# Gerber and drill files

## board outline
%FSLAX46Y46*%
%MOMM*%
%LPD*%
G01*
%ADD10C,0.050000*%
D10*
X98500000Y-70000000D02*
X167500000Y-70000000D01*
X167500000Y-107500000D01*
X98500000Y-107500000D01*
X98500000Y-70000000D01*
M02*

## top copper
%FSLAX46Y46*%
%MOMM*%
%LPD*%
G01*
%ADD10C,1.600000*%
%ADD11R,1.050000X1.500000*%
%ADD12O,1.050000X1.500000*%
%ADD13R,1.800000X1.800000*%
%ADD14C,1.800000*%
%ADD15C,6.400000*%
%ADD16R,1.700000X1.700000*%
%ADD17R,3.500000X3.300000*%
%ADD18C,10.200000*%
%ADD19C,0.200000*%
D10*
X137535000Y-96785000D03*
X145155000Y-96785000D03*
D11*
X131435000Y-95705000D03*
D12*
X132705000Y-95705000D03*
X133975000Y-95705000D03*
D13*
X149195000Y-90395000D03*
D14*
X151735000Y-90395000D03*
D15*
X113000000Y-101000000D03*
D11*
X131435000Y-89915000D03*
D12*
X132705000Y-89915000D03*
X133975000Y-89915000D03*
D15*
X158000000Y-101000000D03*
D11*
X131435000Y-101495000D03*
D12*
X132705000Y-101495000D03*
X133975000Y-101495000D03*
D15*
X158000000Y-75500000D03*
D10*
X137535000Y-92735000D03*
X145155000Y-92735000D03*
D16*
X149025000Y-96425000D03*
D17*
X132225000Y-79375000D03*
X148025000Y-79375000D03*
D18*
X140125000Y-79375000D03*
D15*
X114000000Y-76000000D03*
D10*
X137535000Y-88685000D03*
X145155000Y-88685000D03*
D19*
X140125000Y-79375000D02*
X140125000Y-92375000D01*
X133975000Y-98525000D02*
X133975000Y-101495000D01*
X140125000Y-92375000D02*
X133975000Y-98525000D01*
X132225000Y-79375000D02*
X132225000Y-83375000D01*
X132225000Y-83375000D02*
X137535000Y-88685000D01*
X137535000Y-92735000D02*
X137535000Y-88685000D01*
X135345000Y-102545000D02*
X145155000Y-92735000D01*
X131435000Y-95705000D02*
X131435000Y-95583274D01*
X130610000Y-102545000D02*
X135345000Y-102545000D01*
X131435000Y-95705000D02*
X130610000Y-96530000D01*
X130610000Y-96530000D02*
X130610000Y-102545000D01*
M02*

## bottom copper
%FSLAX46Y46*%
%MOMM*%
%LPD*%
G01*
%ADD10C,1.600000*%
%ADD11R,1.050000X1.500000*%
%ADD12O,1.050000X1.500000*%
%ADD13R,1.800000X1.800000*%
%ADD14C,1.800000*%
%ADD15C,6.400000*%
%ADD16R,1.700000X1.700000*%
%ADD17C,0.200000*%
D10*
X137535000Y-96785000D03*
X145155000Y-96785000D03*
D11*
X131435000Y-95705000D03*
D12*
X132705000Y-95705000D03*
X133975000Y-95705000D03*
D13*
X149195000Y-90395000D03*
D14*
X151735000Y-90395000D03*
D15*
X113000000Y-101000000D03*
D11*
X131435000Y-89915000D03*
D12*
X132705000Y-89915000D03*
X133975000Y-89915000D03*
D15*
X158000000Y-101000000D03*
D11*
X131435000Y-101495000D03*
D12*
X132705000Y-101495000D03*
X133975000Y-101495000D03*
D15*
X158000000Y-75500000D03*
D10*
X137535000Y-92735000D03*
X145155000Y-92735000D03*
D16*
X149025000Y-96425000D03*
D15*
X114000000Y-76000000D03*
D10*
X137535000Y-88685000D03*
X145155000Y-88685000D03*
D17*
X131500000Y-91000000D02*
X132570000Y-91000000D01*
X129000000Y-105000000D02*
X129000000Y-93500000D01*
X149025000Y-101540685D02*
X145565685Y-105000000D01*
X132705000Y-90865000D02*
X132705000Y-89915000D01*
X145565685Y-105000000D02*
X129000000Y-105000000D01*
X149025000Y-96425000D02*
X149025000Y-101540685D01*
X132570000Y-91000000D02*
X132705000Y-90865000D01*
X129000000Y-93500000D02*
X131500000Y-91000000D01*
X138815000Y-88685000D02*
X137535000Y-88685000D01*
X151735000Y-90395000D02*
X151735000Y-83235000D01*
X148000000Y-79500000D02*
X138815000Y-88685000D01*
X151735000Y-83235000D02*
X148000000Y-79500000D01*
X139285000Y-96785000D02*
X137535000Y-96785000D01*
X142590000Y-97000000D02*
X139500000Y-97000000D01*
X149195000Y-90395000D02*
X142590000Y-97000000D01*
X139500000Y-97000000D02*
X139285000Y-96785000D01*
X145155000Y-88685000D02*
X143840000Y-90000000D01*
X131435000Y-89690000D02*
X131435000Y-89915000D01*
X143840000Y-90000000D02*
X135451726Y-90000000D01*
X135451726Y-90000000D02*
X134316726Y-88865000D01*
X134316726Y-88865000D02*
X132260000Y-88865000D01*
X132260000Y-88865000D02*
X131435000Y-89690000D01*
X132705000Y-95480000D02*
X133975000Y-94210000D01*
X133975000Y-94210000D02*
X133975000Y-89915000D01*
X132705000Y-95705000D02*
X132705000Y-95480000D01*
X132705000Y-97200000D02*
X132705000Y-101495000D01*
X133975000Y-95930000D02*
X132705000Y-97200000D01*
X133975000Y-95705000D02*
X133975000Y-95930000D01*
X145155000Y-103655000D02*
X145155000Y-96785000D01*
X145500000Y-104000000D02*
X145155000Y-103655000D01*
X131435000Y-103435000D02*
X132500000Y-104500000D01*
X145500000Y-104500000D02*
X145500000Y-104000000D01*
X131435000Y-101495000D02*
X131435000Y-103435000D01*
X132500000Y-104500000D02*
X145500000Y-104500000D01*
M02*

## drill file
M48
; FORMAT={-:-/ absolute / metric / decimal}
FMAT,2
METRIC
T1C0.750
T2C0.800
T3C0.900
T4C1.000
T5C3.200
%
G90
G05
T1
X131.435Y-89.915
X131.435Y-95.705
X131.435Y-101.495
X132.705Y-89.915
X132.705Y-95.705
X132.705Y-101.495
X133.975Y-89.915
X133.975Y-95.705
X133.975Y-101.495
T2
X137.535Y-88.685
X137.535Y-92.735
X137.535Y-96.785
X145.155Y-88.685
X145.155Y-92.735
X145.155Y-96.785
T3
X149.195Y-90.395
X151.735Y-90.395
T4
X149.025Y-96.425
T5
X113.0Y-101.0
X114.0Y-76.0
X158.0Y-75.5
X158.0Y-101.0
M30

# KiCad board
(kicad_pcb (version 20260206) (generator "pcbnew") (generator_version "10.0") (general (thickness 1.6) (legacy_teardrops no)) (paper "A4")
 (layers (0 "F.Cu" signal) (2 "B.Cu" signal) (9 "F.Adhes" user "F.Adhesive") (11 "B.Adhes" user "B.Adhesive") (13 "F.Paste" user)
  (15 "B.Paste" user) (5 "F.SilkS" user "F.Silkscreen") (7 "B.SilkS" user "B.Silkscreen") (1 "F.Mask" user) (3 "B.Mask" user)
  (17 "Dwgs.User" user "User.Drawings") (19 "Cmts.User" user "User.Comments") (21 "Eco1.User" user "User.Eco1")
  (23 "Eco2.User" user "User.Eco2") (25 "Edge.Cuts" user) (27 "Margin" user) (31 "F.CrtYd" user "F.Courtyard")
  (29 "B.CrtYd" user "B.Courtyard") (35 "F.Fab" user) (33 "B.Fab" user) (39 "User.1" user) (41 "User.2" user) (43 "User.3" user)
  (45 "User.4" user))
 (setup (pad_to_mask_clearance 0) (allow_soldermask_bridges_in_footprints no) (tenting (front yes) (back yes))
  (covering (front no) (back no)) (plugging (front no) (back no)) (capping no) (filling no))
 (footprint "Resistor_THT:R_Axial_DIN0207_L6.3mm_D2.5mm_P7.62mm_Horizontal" (layer "F.Cu") (at 137.535 96.785)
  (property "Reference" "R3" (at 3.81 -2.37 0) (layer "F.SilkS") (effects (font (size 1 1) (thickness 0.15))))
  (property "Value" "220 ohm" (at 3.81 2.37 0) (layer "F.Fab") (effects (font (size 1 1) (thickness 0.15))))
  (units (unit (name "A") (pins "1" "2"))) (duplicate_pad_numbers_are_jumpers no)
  (pad "1" thru_hole circle (at 0 0) (size 1.6 1.6) (drill 0.8) (layers "*.Cu" "*.Mask") (remove_unused_layers no) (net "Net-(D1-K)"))
  (pad "2" thru_hole circle (at 7.62 0) (size 1.6 1.6) (drill 0.8) (layers "*.Cu" "*.Mask") (remove_unused_layers no) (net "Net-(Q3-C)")))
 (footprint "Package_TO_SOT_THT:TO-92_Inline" (layer "F.Cu") (at 131.435 95.705)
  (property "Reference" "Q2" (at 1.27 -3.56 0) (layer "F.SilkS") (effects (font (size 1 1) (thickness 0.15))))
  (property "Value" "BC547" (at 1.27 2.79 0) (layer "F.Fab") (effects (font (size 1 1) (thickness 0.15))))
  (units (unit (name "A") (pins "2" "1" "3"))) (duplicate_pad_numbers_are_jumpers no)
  (pad "1" thru_hole rect (at 0 0) (size 1.05 1.5) (drill 0.75) (layers "*.Cu" "*.Mask") (remove_unused_layers no) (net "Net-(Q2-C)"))
  (pad "2" thru_hole oval (at 1.27 0) (size 1.05 1.5) (drill 0.75) (layers "*.Cu" "*.Mask") (remove_unused_layers no) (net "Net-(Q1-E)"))
  (pad "3" thru_hole oval (at 2.54 0) (size 1.05 1.5) (drill 0.75) (layers "*.Cu" "*.Mask") (remove_unused_layers no) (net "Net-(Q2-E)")))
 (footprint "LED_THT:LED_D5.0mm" (layer "F.Cu") (at 149.195 90.395)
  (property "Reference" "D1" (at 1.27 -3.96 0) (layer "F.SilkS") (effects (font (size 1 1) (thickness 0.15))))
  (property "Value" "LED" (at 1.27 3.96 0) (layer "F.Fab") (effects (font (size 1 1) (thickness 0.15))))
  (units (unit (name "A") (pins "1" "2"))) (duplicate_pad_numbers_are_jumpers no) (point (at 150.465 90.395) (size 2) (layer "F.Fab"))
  (pad "1" thru_hole rect (at 0 0) (size 1.8 1.8) (drill 0.9) (layers "*.Cu" "*.Mask") (remove_unused_layers no) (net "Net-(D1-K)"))
  (pad "2" thru_hole circle (at 2.54 0) (size 1.8 1.8) (drill 0.9) (layers "*.Cu" "*.Mask") (remove_unused_layers no) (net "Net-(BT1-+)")))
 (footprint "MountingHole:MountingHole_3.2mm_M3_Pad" (layer "F.Cu") (at 113 101)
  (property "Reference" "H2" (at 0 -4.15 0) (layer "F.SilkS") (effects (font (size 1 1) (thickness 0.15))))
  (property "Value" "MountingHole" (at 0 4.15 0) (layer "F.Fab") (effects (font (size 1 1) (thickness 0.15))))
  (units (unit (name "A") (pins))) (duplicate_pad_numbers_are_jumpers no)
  (pad "1" thru_hole circle (at 0 0) (size 6.4 6.4) (drill 3.2) (layers "*.Cu" "*.Mask") (remove_unused_layers no) (zone_connect 2)))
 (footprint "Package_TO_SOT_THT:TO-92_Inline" (layer "F.Cu") (at 131.435 89.915)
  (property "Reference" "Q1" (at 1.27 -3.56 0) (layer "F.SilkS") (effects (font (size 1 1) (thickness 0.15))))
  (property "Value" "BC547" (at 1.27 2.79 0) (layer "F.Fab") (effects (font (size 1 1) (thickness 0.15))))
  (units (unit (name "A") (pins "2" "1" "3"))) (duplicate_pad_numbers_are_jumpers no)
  (pad "1" thru_hole rect (at 0 0) (size 1.05 1.5) (drill 0.75) (layers "*.Cu" "*.Mask") (remove_unused_layers no) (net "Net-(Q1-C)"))
  (pad "2" thru_hole oval (at 1.27 0) (size 1.05 1.5) (drill 0.75) (layers "*.Cu" "*.Mask") (remove_unused_layers no) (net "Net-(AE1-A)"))
  (pad "3" thru_hole oval (at 2.54 0) (size 1.05 1.5) (drill 0.75) (layers "*.Cu" "*.Mask") (remove_unused_layers no) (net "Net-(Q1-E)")))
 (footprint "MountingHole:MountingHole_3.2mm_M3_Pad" (layer "F.Cu") (at 158 101)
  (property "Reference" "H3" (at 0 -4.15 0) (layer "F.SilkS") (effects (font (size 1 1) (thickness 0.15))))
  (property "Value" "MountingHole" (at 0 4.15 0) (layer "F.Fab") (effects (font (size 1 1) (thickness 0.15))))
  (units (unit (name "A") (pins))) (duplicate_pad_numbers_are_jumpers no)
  (pad "1" thru_hole circle (at 0 0) (size 6.4 6.4) (drill 3.2) (layers "*.Cu" "*.Mask") (remove_unused_layers no) (zone_connect 2)))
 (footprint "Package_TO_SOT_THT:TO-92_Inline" (layer "F.Cu") (at 131.435 101.495)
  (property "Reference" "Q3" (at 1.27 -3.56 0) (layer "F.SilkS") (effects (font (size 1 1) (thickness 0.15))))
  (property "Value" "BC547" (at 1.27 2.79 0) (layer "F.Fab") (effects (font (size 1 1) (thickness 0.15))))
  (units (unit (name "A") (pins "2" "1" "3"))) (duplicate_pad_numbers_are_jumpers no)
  (pad "1" thru_hole rect (at 0 0) (size 1.05 1.5) (drill 0.75) (layers "*.Cu" "*.Mask") (remove_unused_layers no) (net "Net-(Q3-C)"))
  (pad "2" thru_hole oval (at 1.27 0) (size 1.05 1.5) (drill 0.75) (layers "*.Cu" "*.Mask") (remove_unused_layers no) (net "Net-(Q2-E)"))
  (pad "3" thru_hole oval (at 2.54 0) (size 1.05 1.5) (drill 0.75) (layers "*.Cu" "*.Mask") (remove_unused_layers no) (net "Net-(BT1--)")))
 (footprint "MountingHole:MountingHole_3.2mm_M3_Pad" (layer "F.Cu") (at 158 75.5)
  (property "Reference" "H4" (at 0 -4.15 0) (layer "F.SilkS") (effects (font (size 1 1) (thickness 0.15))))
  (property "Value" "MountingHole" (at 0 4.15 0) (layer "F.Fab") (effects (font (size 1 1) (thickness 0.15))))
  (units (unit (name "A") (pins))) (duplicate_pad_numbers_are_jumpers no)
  (pad "1" thru_hole circle (at 0 0) (size 6.4 6.4) (drill 3.2) (layers "*.Cu" "*.Mask") (remove_unused_layers no) (zone_connect 2)))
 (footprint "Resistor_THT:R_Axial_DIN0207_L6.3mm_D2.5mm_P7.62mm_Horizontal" (layer "F.Cu") (at 137.535 92.735)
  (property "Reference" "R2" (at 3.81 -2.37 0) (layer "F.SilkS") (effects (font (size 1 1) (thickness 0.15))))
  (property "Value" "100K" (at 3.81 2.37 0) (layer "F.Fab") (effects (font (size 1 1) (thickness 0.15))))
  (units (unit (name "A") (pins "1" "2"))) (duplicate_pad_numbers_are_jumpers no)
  (pad "1" thru_hole circle (at 0 0) (size 1.6 1.6) (drill 0.8) (layers "*.Cu" "*.Mask") (remove_unused_layers no) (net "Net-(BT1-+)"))
  (pad "2" thru_hole circle (at 7.62 0) (size 1.6 1.6) (drill 0.8) (layers "*.Cu" "*.Mask") (remove_unused_layers no) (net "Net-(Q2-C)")))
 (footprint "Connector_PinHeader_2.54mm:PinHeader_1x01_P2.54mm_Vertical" (layer "F.Cu") (at 149.025 96.425)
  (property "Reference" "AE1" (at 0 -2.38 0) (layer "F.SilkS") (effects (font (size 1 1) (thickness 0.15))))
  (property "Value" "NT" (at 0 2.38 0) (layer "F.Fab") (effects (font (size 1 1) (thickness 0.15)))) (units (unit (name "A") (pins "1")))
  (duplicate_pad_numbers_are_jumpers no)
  (pad "1" thru_hole rect (at 0 0) (size 1.7 1.7) (drill 1) (layers "*.Cu" "*.Mask") (remove_unused_layers no) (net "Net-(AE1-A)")))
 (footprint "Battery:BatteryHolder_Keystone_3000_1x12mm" (layer "F.Cu") (at 140.125 79.375)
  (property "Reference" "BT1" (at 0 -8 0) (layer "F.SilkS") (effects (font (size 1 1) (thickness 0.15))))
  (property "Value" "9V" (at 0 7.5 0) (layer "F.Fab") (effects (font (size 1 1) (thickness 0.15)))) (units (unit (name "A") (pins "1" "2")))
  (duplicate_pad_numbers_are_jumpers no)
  (pad "1" smd rect (at -7.9 0) (size 3.5 3.3) (layers "F.Cu" "F.Mask" "F.Paste") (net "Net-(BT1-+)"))
  (pad "1" smd rect (at 7.9 0) (size 3.5 3.3) (layers "F.Cu" "F.Mask" "F.Paste") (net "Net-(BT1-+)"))
  (pad "2" smd circle (at 0 0) (size 10.2 10.2) (layers "F.Cu" "F.Mask") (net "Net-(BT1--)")))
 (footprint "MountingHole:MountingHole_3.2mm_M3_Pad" (layer "F.Cu") (at 114 76)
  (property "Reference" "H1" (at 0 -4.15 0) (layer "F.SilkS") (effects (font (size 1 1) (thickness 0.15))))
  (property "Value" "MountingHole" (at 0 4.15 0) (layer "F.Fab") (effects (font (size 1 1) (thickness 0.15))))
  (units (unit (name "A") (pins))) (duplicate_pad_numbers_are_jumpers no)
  (pad "1" thru_hole circle (at 0 0) (size 6.4 6.4) (drill 3.2) (layers "*.Cu" "*.Mask") (remove_unused_layers no) (zone_connect 2)))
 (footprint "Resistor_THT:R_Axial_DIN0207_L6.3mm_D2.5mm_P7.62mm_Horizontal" (layer "F.Cu") (at 137.535 88.685)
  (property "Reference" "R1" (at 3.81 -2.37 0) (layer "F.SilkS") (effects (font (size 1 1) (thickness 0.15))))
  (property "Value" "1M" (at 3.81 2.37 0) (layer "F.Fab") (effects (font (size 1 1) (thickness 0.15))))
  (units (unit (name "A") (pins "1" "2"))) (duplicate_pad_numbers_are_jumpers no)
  (pad "1" thru_hole circle (at 0 0) (size 1.6 1.6) (drill 0.8) (layers "*.Cu" "*.Mask") (remove_unused_layers no) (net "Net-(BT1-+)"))
  (pad "2" thru_hole circle (at 7.62 0) (size 1.6 1.6) (drill 0.8) (layers "*.Cu" "*.Mask") (remove_unused_layers no) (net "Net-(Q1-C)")))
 (gr_rect (start 98.5 70) (end 167.5 107.5) (stroke (width 0.05) (type default)) (fill no) (layer "Edge.Cuts"))
 (segment (start 131.5 91) (end 132.57 91) (width 0.2) (layer "B.Cu") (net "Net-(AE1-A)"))
 (segment (start 129 105) (end 129 93.5) (width 0.2) (layer "B.Cu") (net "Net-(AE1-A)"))
 (segment (start 149.025 101.540685) (end 145.565685 105) (width 0.2) (layer "B.Cu") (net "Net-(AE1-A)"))
 (segment (start 132.705 90.865) (end 132.705 89.915) (width 0.2) (layer "B.Cu") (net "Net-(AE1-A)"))
 (segment (start 145.565685 105) (end 129 105) (width 0.2) (layer "B.Cu") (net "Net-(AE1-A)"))
 (segment (start 149.025 96.425) (end 149.025 101.540685) (width 0.2) (layer "B.Cu") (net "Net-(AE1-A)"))
 (segment (start 132.57 91) (end 132.705 90.865) (width 0.2) (layer "B.Cu") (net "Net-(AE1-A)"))
 (segment (start 129 93.5) (end 131.5 91) (width 0.2) (layer "B.Cu") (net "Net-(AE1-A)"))
 (segment (start 140.125 79.375) (end 140.125 92.375) (width 0.2) (layer "F.Cu") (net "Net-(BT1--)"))
 (segment (start 133.975 98.525) (end 133.975 101.495) (width 0.2) (layer "F.Cu") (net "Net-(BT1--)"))
 (segment (start 140.125 92.375) (end 133.975 98.525) (width 0.2) (layer "F.Cu") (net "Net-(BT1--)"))
 (segment (start 132.225 79.375) (end 132.225 83.375) (width 0.2) (layer "F.Cu") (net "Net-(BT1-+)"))
 (segment (start 132.225 83.375) (end 137.535 88.685) (width 0.2) (layer "F.Cu") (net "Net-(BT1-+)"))
 (segment (start 137.535 92.735) (end 137.535 88.685) (width 0.2) (layer "F.Cu") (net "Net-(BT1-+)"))
 (segment (start 138.815 88.685) (end 137.535 88.685) (width 0.2) (layer "B.Cu") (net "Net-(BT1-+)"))
 (segment (start 151.735 90.395) (end 151.735 83.235) (width 0.2) (layer "B.Cu") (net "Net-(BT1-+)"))
 (segment (start 148 79.5) (end 138.815 88.685) (width 0.2) (layer "B.Cu") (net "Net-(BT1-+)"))
 (segment (start 151.735 83.235) (end 148 79.5) (width 0.2) (layer "B.Cu") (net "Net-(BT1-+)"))
 (segment (start 139.285 96.785) (end 137.535 96.785) (width 0.2) (layer "B.Cu") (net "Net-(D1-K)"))
 (segment (start 142.59 97) (end 139.5 97) (width 0.2) (layer "B.Cu") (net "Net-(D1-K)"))
 (segment (start 149.195 90.395) (end 142.59 97) (width 0.2) (layer "B.Cu") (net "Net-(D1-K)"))
 (segment (start 139.5 97) (end 139.285 96.785) (width 0.2) (layer "B.Cu") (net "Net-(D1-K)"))
 (segment (start 145.155 88.685) (end 143.84 90) (width 0.2) (layer "B.Cu") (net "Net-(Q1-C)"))
 (segment (start 131.435 89.69) (end 131.435 89.915) (width 0.2) (layer "B.Cu") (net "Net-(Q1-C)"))
 (segment (start 143.84 90) (end 135.451726 90) (width 0.2) (layer "B.Cu") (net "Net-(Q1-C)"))
 (segment (start 135.451726 90) (end 134.316726 88.865) (width 0.2) (layer "B.Cu") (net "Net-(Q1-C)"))
 (segment (start 134.316726 88.865) (end 132.26 88.865) (width 0.2) (layer "B.Cu") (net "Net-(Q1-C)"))
 (segment (start 132.26 88.865) (end 131.435 89.69) (width 0.2) (layer "B.Cu") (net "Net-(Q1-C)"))
 (segment (start 132.705 95.48) (end 133.975 94.21) (width 0.2) (layer "B.Cu") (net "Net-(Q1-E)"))
 (segment (start 133.975 94.21) (end 133.975 89.915) (width 0.2) (layer "B.Cu") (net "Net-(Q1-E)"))
 (segment (start 132.705 95.705) (end 132.705 95.48) (width 0.2) (layer "B.Cu") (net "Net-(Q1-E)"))
 (segment (start 135.345 102.545) (end 145.155 92.735) (width 0.2) (layer "F.Cu") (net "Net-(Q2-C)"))
 (segment (start 131.435 95.705) (end 131.435 95.583274) (width 0.2) (layer "F.Cu") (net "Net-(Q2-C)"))
 (segment (start 130.61 102.545) (end 135.345 102.545) (width 0.2) (layer "F.Cu") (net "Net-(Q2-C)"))
 (segment (start 131.435 95.705) (end 130.61 96.53) (width 0.2) (layer "F.Cu") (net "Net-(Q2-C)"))
 (segment (start 130.61 96.53) (end 130.61 102.545) (width 0.2) (layer "F.Cu") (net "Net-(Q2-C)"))
 (segment (start 132.705 97.2) (end 132.705 101.495) (width 0.2) (layer "B.Cu") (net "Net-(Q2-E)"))
 (segment (start 133.975 95.93) (end 132.705 97.2) (width 0.2) (layer "B.Cu") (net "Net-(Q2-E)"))
 (segment (start 133.975 95.705) (end 133.975 95.93) (width 0.2) (layer "B.Cu") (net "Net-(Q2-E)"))
 (segment (start 145.155 103.655) (end 145.155 96.785) (width 0.2) (layer "B.Cu") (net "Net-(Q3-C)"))
 (segment (start 145.5 104) (end 145.155 103.655) (width 0.2) (layer "B.Cu") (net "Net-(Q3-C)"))
 (segment (start 131.435 103.435) (end 132.5 104.5) (width 0.2) (layer "B.Cu") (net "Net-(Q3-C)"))
 (segment (start 145.5 104.5) (end 145.5 104) (width 0.2) (layer "B.Cu") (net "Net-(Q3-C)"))
 (segment (start 131.435 101.495) (end 131.435 103.435) (width 0.2) (layer "B.Cu") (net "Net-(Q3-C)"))
 (segment (start 132.5 104.5) (end 145.5 104.5) (width 0.2) (layer "B.Cu") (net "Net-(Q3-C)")))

